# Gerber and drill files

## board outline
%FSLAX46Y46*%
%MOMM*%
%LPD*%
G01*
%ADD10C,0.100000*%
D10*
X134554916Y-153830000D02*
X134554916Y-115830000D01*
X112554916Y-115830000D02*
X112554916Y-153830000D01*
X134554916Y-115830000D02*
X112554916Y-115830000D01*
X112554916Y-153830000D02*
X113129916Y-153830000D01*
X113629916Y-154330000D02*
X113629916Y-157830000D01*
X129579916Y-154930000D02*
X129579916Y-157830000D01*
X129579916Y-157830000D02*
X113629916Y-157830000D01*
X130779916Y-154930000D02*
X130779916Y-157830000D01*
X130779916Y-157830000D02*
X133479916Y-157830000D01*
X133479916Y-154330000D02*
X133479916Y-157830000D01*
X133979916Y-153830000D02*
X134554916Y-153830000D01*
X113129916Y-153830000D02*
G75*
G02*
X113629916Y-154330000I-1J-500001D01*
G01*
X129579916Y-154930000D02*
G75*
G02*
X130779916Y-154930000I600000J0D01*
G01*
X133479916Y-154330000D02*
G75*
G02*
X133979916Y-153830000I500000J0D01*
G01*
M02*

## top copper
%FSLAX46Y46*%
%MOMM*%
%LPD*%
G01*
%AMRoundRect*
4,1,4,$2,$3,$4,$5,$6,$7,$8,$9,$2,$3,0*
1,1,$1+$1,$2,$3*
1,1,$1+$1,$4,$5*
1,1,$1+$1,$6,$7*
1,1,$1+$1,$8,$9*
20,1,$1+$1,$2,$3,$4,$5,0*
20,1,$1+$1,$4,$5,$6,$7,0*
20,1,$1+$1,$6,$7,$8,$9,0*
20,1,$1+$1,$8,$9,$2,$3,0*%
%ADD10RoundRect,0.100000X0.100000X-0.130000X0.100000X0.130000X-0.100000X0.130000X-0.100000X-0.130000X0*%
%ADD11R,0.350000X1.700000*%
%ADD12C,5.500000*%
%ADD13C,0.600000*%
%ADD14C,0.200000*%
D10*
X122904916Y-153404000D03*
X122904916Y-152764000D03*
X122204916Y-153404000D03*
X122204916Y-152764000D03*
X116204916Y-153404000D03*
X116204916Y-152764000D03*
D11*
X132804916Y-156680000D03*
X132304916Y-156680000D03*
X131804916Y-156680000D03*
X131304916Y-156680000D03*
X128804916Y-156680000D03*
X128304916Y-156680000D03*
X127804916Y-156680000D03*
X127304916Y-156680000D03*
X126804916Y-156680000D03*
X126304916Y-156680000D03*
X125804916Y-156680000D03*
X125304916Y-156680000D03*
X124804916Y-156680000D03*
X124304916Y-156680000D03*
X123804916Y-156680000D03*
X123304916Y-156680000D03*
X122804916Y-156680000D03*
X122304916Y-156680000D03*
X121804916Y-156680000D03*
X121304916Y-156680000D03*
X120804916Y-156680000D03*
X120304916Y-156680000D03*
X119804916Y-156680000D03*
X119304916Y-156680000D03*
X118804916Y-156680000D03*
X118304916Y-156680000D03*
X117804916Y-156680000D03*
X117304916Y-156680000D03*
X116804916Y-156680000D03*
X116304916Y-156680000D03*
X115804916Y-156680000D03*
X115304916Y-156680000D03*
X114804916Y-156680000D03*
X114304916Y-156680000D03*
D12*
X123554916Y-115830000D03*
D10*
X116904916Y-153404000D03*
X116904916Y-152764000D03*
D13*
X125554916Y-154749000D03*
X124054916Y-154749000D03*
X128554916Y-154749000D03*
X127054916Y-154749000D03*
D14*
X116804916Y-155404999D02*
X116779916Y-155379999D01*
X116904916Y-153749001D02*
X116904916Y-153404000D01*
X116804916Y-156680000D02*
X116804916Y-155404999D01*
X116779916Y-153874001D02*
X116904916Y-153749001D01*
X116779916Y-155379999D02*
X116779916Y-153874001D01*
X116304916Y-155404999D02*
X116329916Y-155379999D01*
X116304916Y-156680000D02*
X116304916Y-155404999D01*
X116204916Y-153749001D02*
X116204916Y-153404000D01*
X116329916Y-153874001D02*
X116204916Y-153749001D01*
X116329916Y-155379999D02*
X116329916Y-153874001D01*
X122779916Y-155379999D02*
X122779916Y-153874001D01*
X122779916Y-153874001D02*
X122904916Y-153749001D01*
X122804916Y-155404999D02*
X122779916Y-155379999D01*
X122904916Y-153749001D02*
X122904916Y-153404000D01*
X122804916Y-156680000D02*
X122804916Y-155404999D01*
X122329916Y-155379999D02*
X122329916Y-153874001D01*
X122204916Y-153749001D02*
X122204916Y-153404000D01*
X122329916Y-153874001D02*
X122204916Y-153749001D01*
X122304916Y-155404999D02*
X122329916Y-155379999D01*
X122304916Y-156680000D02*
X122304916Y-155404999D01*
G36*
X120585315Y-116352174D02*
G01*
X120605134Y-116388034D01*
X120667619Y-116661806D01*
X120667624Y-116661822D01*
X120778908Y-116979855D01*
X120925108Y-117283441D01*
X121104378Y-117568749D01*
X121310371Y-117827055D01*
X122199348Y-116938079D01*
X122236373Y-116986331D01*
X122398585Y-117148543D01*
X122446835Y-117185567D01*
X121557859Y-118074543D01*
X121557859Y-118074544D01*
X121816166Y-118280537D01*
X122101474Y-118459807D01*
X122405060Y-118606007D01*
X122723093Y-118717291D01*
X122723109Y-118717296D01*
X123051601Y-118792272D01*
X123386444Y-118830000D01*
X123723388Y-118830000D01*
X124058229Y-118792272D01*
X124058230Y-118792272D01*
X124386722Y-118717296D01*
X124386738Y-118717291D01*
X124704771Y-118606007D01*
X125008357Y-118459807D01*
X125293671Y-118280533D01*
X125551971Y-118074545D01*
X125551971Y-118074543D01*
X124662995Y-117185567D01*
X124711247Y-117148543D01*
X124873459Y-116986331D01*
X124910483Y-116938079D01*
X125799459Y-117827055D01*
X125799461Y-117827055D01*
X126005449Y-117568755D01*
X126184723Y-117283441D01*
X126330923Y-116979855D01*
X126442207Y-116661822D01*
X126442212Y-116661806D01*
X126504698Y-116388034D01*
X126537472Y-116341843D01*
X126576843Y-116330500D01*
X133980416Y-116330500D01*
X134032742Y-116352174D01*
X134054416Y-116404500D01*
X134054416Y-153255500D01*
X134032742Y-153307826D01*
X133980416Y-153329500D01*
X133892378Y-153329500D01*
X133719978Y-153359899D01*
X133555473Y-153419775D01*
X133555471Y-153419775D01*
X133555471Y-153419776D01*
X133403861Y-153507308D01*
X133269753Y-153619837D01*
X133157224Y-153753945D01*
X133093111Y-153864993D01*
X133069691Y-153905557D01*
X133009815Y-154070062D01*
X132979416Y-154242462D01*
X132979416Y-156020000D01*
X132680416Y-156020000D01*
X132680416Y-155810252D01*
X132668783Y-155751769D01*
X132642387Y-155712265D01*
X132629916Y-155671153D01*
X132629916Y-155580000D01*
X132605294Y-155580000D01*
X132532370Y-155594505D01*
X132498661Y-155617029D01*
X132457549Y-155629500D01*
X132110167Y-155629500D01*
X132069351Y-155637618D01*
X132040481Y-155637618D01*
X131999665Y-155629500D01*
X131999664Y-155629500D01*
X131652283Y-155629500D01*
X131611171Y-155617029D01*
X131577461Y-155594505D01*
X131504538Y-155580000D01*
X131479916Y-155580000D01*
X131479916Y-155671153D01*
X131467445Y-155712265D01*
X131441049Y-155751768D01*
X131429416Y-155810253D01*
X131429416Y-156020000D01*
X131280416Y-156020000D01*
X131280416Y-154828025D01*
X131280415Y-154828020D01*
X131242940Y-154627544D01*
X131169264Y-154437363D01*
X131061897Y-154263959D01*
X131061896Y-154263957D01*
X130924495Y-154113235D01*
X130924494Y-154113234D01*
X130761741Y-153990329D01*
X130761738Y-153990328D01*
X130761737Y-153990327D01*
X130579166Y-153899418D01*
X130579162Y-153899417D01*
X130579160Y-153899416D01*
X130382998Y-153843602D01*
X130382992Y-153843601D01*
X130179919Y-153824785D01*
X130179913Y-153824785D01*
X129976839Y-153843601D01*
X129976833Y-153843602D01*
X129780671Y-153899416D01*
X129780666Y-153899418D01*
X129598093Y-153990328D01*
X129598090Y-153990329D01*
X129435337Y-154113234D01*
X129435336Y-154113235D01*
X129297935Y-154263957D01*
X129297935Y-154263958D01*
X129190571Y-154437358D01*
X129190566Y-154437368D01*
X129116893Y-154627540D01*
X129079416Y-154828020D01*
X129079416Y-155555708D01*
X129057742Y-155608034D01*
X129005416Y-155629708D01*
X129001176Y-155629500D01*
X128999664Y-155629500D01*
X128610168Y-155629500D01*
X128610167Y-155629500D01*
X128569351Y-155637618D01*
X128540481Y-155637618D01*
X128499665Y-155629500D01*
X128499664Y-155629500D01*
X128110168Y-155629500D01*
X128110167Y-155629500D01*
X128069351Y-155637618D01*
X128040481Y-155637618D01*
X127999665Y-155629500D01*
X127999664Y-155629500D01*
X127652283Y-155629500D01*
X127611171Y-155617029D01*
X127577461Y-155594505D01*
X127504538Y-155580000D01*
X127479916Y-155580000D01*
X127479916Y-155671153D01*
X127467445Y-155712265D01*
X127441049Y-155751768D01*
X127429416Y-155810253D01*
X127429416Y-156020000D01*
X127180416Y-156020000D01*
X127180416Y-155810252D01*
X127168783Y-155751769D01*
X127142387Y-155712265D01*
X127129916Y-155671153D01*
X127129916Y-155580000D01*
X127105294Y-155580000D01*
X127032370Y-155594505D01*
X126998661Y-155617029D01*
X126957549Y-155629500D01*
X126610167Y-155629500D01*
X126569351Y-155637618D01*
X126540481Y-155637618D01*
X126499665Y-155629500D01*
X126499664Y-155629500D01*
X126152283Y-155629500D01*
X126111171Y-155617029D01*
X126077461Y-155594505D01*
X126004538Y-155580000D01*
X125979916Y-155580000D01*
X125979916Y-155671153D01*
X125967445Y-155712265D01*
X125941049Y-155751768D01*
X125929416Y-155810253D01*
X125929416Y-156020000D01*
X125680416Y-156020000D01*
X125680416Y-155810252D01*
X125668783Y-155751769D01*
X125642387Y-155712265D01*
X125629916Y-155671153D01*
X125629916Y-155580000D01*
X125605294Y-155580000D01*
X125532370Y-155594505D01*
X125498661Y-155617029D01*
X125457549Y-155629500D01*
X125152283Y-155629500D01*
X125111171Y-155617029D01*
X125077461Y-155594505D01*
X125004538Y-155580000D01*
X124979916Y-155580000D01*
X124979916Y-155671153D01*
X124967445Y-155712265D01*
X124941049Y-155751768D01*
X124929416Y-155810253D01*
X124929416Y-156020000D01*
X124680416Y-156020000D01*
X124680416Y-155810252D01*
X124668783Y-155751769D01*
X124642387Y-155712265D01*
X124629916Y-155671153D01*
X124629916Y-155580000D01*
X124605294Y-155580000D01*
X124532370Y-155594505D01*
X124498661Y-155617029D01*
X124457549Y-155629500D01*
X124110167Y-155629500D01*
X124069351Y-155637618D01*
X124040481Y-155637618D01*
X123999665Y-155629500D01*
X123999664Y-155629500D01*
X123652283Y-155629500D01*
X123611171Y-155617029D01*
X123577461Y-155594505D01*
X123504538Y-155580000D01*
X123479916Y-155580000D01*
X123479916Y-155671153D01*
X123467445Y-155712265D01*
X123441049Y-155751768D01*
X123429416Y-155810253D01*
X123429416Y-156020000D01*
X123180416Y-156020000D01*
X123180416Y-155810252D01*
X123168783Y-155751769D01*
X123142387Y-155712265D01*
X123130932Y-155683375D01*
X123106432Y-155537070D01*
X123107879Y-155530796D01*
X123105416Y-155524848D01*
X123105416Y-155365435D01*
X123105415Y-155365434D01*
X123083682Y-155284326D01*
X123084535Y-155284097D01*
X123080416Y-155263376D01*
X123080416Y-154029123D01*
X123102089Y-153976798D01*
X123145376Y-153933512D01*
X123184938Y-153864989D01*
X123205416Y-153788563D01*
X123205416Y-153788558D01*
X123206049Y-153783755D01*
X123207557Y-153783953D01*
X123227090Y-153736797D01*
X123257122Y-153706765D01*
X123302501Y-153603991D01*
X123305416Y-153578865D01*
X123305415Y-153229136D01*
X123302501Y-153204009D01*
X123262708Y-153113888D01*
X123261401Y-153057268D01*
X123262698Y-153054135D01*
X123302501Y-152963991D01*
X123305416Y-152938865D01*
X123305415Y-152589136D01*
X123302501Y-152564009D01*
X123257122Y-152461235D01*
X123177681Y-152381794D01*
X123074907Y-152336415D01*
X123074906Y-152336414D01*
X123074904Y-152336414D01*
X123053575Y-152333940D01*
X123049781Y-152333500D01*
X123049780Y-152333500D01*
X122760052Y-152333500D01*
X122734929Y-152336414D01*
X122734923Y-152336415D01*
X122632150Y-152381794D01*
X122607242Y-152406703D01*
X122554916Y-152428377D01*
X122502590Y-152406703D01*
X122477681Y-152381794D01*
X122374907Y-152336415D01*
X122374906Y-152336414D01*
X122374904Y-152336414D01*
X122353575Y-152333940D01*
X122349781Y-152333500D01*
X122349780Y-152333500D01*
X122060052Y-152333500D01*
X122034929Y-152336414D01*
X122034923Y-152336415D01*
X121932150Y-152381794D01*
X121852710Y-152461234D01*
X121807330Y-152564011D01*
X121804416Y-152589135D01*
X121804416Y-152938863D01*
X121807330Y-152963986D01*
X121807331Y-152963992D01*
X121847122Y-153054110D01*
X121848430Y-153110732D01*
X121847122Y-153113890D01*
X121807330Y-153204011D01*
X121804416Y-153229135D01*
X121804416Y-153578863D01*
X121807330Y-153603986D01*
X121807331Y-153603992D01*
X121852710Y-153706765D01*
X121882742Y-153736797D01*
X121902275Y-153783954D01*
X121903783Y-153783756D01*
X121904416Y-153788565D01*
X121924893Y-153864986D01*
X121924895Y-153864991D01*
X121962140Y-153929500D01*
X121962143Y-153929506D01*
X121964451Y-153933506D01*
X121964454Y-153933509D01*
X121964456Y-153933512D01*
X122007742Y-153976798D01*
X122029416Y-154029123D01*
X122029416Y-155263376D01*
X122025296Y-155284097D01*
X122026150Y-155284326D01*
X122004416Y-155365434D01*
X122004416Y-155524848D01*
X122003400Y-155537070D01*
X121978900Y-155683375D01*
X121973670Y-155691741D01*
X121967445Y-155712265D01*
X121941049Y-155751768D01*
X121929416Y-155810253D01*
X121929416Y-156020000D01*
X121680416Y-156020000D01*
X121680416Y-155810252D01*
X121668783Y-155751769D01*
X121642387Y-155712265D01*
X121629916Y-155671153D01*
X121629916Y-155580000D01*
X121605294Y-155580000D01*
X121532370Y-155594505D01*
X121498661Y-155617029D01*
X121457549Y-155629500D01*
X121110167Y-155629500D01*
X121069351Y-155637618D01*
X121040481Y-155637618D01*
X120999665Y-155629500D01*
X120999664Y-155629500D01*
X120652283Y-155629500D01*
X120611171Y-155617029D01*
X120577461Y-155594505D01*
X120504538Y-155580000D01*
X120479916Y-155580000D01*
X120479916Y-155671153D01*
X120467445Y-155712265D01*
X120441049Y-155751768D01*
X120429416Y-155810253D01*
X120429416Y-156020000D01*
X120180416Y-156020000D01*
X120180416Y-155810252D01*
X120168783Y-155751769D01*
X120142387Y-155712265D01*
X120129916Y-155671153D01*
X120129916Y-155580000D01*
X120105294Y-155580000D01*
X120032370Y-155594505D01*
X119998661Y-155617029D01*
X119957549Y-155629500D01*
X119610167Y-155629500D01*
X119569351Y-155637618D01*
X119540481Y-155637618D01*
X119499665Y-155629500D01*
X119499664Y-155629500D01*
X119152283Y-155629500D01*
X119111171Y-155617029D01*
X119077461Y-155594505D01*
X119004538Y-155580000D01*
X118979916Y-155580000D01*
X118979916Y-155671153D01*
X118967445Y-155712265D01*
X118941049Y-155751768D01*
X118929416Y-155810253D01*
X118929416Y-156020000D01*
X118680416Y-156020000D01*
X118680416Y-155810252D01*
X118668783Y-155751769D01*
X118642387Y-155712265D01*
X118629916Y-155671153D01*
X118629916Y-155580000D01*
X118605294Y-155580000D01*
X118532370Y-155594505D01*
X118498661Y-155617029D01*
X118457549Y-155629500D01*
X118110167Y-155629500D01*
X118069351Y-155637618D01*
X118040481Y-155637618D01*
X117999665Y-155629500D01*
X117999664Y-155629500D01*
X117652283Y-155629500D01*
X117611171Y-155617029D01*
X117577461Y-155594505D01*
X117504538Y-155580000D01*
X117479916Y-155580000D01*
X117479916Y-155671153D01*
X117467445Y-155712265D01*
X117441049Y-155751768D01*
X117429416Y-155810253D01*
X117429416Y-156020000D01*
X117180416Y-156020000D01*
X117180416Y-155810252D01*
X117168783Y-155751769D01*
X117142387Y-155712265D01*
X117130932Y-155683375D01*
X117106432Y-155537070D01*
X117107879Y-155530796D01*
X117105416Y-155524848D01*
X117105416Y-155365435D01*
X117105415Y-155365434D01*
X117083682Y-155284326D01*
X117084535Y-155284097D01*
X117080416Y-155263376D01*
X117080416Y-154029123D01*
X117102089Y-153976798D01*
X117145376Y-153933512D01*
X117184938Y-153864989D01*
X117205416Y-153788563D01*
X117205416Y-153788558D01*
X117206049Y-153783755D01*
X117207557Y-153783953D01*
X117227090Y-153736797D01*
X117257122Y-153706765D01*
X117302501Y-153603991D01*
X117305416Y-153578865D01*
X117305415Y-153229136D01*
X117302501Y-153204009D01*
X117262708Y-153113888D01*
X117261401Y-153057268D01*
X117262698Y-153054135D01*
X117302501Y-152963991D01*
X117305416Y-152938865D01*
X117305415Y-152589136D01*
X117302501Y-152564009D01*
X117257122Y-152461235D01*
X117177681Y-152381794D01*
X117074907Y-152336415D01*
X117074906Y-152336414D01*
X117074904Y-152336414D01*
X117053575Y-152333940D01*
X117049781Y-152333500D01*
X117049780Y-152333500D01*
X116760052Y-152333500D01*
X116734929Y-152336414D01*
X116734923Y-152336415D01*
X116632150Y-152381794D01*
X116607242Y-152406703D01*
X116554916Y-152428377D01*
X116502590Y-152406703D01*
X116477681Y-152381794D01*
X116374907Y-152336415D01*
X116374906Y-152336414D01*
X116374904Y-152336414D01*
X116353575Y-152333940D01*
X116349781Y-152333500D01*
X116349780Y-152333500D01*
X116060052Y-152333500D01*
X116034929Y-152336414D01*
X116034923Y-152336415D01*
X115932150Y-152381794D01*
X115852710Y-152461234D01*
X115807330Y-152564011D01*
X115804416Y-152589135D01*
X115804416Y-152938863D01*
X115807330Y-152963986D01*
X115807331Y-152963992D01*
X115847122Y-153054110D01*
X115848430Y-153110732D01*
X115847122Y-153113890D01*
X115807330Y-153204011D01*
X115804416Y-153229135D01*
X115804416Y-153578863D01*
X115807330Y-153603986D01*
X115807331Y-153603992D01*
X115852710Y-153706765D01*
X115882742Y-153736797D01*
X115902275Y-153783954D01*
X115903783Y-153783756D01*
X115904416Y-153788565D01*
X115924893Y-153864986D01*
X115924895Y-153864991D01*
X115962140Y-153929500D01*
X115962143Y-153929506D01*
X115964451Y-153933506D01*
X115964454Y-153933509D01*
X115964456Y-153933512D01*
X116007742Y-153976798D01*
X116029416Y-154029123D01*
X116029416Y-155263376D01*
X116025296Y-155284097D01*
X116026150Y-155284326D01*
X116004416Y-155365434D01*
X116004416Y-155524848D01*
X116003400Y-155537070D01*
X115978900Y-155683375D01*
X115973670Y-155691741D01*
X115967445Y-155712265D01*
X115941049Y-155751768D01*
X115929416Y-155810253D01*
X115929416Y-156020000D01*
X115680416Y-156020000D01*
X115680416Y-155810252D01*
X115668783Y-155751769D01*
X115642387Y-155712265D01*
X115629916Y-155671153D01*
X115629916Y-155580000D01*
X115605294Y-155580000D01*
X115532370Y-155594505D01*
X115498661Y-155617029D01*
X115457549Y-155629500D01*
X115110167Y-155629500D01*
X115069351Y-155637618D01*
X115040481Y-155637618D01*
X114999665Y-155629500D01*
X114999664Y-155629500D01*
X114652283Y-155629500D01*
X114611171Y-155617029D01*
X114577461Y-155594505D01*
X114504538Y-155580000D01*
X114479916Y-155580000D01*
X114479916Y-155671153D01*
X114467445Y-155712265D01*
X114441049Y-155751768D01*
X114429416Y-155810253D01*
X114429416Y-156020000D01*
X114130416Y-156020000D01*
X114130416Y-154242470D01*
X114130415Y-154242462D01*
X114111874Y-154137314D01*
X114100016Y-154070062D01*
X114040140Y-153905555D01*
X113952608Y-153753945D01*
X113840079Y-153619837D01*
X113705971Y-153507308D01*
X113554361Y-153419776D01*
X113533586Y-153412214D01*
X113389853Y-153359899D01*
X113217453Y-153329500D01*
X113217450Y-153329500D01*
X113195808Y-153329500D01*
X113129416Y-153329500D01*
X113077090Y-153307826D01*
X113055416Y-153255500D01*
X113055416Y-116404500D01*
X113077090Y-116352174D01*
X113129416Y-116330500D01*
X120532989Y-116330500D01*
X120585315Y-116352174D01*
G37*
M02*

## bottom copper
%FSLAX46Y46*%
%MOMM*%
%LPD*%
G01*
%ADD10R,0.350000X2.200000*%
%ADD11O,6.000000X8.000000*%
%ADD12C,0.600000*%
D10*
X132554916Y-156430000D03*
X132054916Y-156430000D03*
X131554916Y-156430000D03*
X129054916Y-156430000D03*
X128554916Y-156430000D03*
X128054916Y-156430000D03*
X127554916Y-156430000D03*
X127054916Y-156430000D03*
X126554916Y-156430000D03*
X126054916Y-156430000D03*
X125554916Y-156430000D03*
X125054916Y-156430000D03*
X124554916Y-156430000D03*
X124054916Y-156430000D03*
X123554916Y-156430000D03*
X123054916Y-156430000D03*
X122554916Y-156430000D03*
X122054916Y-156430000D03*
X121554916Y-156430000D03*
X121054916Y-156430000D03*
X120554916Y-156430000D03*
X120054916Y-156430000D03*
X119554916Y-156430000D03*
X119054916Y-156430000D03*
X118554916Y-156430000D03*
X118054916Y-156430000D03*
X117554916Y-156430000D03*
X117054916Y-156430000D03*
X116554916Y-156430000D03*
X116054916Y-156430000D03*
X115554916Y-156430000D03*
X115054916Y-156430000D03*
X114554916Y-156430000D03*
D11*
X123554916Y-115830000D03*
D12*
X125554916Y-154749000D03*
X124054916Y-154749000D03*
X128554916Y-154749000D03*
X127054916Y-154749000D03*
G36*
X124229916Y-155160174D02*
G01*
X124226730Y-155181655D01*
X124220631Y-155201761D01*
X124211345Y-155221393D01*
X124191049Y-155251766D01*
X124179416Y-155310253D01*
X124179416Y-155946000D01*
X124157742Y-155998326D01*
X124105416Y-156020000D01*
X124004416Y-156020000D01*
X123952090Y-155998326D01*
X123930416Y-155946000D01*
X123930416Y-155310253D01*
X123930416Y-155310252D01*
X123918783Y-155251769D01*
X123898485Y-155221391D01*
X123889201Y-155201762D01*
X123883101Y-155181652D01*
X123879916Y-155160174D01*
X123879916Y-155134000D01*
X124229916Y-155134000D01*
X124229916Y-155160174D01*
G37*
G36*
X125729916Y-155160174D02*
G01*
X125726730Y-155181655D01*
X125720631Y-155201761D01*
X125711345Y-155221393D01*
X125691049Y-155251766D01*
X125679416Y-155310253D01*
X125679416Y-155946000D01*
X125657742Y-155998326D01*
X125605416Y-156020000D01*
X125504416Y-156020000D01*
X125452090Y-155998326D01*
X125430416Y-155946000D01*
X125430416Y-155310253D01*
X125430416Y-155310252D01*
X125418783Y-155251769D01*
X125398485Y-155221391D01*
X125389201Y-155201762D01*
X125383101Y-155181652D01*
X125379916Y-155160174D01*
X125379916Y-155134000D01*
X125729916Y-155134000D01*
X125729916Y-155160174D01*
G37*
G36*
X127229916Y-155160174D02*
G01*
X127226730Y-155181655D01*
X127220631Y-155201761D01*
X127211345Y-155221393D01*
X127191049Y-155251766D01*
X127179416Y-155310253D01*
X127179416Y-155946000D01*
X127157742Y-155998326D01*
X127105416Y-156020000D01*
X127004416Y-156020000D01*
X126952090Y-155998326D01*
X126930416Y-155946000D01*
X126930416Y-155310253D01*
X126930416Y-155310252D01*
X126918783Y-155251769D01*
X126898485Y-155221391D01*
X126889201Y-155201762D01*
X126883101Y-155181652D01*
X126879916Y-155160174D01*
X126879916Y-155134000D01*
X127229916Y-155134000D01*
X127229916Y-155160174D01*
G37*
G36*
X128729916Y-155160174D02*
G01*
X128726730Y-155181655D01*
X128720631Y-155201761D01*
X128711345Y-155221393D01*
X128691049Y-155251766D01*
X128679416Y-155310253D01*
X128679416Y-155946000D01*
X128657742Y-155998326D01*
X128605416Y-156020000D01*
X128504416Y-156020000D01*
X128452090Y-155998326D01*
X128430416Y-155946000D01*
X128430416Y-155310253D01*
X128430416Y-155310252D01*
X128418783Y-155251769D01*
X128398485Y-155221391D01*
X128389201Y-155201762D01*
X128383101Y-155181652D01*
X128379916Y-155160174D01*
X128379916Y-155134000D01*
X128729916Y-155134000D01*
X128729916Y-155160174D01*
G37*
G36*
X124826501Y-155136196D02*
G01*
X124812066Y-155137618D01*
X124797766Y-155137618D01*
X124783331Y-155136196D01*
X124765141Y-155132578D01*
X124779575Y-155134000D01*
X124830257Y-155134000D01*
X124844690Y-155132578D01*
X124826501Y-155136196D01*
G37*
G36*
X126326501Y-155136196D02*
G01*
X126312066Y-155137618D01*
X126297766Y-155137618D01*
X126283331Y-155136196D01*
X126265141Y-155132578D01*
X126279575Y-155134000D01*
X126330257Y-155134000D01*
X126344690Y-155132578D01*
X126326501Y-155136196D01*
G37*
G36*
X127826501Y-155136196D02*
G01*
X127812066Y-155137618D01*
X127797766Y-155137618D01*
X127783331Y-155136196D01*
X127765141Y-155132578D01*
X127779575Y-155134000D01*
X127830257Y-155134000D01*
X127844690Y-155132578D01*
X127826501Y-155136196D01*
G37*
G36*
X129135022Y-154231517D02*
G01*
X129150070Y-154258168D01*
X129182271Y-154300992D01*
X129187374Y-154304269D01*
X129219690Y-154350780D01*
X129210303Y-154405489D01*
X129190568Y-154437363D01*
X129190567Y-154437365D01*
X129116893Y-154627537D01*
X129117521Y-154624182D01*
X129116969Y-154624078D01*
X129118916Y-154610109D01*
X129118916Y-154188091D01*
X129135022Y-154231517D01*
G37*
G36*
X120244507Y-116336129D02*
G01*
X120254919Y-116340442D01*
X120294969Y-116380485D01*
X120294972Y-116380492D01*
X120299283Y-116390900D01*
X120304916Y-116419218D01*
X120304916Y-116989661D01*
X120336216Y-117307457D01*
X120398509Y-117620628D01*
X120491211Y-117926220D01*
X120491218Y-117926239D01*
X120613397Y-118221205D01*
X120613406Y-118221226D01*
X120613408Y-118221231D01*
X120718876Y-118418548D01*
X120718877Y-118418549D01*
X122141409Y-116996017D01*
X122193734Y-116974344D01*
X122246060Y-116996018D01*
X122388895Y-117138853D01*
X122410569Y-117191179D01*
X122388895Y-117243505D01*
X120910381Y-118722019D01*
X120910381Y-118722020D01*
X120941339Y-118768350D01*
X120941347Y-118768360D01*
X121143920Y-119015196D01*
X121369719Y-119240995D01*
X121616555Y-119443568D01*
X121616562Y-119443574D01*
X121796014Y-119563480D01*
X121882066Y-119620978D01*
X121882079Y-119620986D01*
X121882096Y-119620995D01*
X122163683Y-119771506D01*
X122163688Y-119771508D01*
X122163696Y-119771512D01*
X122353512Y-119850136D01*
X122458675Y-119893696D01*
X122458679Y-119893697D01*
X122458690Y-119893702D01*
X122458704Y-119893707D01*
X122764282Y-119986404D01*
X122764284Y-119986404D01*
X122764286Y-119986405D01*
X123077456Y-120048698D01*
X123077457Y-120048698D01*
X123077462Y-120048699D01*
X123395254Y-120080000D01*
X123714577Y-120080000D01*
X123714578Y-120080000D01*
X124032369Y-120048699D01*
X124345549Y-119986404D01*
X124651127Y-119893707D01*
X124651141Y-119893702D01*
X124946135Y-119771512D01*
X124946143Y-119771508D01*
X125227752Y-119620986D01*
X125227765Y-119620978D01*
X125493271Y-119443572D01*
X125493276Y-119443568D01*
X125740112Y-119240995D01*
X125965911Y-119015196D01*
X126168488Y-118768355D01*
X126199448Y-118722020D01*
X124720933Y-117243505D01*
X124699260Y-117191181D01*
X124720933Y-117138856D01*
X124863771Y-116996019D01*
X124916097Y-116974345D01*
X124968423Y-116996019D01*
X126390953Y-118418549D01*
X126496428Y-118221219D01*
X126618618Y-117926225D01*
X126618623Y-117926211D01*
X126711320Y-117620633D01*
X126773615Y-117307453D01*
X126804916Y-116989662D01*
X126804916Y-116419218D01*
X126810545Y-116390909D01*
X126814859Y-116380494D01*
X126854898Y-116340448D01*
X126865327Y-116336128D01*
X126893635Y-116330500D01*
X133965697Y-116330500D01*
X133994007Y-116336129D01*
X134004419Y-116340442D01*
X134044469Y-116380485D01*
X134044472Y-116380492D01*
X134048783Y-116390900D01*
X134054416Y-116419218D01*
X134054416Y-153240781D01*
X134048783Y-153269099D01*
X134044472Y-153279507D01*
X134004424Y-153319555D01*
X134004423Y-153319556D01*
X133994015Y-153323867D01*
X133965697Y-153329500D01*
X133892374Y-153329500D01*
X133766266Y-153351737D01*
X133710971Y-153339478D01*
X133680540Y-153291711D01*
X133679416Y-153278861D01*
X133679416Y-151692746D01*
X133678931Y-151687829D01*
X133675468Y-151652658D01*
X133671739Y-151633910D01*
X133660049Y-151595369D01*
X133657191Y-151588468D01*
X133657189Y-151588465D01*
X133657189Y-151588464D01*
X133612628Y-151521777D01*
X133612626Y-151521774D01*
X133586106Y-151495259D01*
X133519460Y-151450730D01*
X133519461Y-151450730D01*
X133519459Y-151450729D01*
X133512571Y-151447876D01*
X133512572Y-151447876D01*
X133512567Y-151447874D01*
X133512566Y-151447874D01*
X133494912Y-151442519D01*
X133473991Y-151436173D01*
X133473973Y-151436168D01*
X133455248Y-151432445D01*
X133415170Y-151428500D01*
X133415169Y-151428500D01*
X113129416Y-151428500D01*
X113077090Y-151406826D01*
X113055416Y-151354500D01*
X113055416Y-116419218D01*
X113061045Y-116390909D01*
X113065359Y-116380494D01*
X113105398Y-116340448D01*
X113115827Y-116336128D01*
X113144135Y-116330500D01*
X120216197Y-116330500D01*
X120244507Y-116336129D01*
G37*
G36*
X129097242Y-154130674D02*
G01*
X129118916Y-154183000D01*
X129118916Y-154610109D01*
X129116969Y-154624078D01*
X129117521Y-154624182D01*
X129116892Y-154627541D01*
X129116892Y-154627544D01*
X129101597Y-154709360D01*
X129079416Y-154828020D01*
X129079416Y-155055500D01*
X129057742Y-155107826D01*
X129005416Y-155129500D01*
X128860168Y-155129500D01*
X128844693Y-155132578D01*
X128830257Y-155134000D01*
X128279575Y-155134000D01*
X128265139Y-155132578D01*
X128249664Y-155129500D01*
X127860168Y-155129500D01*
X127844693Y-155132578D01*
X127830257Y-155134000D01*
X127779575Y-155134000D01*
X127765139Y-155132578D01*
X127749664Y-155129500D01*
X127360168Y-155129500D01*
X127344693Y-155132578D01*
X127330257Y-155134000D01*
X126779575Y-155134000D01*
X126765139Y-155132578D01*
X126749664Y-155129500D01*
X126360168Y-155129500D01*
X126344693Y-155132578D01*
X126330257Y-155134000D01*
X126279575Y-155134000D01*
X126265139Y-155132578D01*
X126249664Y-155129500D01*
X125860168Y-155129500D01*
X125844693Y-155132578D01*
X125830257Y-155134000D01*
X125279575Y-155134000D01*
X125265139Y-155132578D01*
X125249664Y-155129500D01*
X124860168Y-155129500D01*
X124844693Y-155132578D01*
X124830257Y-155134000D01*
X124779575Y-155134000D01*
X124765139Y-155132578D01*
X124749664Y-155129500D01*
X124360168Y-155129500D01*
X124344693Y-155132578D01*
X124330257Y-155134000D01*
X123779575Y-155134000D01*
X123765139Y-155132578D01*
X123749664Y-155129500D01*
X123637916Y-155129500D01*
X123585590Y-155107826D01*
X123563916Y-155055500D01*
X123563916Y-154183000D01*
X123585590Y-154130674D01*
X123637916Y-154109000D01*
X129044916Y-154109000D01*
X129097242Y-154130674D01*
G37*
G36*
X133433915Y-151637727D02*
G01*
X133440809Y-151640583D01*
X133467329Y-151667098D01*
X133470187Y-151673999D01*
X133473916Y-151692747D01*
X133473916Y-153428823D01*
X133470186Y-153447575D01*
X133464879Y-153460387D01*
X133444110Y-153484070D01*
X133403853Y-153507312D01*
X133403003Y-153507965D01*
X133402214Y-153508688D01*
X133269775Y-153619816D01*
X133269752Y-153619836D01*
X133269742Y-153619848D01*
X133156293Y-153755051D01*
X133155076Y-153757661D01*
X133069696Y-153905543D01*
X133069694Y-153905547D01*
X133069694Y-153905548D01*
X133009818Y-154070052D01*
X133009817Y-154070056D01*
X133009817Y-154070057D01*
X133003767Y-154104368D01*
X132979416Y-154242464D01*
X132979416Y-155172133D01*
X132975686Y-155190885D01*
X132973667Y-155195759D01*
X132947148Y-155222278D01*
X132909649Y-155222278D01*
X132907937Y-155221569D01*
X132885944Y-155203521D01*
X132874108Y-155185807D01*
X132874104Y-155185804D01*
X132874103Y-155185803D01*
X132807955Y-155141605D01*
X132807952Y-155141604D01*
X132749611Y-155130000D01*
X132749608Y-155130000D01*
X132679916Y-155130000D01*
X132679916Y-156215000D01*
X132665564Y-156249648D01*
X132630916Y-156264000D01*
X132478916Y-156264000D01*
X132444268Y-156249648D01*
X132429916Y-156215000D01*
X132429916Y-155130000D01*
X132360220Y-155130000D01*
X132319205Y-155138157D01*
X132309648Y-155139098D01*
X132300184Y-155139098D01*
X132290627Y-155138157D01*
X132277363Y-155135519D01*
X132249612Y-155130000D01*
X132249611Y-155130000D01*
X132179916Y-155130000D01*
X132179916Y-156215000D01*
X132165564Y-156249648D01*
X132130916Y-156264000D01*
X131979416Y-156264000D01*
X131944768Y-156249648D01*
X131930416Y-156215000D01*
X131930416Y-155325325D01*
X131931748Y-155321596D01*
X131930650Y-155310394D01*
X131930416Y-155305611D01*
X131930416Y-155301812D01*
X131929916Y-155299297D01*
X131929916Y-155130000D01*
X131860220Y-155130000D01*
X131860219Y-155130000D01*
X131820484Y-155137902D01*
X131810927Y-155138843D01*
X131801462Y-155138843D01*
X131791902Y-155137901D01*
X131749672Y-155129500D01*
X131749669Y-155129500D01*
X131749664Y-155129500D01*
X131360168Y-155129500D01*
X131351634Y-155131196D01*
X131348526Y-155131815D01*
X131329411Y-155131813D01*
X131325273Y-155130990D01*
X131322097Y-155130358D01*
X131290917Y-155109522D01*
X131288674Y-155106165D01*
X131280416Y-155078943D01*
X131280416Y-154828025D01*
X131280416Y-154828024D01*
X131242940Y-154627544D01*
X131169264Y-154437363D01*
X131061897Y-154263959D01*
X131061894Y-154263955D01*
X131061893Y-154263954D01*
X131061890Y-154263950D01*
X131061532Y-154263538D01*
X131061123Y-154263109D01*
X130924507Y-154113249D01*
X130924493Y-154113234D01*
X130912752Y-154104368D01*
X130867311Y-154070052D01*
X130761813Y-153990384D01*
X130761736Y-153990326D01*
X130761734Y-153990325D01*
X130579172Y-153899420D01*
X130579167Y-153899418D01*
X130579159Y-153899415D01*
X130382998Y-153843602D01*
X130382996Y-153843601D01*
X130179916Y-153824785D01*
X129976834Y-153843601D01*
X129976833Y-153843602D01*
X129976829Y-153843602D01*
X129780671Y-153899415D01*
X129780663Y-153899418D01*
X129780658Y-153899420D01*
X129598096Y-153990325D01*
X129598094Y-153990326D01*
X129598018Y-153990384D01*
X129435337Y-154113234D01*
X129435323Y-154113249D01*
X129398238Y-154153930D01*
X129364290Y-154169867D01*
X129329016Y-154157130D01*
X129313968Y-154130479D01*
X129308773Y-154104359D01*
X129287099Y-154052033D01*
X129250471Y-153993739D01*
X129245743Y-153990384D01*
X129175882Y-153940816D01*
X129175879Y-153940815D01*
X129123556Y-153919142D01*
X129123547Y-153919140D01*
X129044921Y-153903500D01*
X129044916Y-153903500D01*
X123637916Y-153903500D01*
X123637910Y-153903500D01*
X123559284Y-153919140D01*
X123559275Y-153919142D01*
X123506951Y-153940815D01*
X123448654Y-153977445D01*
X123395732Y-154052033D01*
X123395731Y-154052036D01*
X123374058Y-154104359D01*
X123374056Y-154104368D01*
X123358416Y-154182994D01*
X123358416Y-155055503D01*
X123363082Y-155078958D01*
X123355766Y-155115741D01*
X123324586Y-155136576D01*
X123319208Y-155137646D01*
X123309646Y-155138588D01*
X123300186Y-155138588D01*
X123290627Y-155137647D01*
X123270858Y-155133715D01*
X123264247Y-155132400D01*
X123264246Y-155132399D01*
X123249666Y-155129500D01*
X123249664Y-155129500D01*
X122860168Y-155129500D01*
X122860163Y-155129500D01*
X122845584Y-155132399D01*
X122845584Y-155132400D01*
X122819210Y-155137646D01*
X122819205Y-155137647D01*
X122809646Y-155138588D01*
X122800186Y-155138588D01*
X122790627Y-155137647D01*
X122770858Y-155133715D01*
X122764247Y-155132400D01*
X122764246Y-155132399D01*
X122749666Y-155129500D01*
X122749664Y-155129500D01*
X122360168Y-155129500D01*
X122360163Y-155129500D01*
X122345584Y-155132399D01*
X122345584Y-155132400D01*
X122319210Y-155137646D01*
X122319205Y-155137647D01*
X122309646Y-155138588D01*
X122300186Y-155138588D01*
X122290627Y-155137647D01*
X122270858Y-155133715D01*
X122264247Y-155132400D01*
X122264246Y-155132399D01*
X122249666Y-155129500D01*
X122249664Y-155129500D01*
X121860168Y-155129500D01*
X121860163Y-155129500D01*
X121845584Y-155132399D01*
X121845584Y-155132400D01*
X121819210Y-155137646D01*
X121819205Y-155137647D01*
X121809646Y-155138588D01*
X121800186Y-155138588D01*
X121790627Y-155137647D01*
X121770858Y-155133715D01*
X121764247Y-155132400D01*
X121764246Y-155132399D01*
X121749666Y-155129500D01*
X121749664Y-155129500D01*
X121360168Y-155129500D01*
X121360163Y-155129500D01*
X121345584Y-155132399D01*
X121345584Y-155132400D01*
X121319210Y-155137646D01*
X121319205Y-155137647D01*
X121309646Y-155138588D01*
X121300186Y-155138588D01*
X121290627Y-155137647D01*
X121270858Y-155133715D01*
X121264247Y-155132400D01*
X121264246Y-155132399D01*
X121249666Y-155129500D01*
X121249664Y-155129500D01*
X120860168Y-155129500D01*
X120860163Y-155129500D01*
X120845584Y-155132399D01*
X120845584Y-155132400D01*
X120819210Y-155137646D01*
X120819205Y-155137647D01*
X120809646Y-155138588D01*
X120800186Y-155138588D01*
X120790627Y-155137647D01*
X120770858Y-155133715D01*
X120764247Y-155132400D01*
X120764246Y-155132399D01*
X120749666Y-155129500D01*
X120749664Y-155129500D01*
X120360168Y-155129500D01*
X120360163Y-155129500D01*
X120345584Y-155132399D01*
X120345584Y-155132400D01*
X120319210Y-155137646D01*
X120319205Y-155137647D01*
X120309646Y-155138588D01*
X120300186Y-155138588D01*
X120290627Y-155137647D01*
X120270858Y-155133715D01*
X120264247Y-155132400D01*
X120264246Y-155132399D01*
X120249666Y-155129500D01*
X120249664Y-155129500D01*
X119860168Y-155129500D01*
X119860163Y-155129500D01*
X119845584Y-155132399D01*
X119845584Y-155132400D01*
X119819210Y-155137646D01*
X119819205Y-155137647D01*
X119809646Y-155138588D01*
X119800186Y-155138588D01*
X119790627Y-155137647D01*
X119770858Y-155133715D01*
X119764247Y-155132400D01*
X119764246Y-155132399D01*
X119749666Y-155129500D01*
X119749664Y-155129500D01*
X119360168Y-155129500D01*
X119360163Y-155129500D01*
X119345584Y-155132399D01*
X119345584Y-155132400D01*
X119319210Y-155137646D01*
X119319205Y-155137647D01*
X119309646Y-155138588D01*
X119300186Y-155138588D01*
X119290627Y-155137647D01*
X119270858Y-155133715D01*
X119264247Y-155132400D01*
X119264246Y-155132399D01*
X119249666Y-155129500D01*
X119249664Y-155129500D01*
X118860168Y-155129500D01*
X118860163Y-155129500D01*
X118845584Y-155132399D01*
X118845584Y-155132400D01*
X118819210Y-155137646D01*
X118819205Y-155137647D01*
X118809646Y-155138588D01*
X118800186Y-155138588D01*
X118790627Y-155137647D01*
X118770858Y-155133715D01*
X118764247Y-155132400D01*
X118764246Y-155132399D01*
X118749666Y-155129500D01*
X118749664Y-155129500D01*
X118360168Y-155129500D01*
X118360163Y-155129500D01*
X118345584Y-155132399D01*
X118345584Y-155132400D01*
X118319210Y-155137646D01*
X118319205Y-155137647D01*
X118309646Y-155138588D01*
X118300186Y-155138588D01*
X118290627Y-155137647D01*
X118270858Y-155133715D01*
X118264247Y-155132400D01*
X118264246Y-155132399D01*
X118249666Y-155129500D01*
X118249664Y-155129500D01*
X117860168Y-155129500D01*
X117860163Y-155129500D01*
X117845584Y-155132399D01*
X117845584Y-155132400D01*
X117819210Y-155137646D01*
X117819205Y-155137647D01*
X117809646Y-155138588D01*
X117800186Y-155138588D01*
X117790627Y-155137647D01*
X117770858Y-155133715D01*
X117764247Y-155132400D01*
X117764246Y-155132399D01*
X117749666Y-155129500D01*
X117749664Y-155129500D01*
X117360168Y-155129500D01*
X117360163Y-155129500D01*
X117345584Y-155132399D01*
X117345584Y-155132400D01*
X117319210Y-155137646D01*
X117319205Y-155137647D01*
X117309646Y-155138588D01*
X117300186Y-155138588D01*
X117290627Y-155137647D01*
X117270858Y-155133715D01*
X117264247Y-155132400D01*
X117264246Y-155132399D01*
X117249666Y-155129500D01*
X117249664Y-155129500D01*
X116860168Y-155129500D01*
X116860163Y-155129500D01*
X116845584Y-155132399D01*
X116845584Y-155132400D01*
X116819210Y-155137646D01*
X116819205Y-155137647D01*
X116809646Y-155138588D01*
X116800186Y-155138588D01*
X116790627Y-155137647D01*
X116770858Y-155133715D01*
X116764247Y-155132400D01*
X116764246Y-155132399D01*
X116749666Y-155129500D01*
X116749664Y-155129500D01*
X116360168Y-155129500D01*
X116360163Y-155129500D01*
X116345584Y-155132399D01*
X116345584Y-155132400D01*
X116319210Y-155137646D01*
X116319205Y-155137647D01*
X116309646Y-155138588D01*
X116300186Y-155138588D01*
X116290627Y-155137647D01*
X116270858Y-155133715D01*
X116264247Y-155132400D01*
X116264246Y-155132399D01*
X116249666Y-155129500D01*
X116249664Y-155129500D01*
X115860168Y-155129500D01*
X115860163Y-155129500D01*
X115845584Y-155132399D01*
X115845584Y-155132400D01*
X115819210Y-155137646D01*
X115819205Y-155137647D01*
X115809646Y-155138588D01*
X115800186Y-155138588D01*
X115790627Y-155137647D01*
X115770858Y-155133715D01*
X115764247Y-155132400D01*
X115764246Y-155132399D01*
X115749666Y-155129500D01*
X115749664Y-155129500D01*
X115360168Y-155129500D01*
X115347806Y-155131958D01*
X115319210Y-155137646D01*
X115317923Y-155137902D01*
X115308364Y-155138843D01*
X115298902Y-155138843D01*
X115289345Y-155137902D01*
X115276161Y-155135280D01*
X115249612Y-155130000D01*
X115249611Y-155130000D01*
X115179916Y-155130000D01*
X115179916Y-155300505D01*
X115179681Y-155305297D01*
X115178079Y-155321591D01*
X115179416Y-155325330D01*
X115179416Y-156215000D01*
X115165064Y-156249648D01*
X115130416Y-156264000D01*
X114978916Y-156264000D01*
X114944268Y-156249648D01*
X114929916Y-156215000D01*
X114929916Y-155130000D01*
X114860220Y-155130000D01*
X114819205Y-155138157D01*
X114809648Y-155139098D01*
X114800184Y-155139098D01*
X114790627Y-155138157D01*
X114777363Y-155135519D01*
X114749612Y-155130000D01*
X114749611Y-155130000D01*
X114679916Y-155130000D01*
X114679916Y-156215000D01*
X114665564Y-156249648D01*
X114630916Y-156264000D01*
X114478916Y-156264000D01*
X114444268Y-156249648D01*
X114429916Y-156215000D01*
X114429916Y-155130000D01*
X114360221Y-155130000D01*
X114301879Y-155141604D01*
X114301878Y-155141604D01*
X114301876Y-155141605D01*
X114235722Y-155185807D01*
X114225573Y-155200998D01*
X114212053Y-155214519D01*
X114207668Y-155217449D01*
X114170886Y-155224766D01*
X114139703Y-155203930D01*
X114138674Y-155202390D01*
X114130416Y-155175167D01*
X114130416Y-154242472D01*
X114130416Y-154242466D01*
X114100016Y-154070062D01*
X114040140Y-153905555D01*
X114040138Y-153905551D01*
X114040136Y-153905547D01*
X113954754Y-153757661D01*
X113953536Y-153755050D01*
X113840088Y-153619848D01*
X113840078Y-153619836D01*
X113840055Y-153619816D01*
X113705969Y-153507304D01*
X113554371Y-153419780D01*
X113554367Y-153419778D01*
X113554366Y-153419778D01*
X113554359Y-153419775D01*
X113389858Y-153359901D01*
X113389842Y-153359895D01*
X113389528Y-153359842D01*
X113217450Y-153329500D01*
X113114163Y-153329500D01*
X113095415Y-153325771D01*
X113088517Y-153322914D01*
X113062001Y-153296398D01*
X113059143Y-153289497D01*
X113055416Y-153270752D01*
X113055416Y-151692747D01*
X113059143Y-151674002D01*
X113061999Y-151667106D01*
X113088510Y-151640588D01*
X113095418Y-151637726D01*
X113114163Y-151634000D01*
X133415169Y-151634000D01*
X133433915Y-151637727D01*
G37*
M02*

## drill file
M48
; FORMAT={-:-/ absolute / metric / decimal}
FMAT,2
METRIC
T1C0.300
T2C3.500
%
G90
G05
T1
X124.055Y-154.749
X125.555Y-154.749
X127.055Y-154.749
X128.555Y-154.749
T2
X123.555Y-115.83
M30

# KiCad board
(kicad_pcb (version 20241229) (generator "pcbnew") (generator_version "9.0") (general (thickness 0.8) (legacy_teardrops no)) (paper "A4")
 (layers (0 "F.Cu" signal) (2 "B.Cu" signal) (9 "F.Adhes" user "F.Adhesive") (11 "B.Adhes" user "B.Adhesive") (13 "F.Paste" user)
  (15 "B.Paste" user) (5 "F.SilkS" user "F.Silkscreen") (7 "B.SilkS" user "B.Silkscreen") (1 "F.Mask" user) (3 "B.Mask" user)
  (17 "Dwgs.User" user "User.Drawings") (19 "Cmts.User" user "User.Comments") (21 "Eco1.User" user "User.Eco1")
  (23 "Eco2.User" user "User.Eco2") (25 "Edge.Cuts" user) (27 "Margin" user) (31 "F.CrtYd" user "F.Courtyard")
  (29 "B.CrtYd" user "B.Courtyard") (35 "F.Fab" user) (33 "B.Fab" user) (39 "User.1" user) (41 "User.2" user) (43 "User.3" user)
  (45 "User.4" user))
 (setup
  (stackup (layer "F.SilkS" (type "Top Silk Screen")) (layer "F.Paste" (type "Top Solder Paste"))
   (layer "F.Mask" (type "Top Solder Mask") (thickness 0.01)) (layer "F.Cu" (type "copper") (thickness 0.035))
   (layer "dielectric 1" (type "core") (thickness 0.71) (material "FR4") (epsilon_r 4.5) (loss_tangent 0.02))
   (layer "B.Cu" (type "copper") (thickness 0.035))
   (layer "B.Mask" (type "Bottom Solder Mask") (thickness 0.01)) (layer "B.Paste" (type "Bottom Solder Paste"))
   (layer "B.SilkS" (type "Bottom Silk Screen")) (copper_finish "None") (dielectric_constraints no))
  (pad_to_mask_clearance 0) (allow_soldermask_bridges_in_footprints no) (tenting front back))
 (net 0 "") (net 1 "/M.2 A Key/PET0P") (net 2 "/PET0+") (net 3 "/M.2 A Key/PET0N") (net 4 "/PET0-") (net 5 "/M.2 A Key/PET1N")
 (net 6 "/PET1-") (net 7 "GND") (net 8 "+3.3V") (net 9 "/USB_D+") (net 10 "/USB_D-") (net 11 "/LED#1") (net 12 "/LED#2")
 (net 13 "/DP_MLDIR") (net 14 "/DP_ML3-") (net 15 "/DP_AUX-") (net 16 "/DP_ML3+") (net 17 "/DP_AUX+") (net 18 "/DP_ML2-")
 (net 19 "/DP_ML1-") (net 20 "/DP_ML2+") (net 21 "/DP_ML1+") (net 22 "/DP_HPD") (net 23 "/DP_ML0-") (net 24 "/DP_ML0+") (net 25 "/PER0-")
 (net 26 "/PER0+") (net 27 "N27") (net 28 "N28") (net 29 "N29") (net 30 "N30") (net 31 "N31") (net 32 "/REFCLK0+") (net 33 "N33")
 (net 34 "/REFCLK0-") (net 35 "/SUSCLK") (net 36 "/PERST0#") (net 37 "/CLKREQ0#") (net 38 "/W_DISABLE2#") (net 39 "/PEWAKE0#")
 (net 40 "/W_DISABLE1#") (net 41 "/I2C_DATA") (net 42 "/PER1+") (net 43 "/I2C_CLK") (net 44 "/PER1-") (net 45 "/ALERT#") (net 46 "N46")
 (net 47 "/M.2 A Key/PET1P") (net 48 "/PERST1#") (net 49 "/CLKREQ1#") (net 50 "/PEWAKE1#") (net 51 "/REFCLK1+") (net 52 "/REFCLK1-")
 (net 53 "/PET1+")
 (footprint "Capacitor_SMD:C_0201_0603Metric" (layer "F.Cu") (at 122.904916 153.084 90)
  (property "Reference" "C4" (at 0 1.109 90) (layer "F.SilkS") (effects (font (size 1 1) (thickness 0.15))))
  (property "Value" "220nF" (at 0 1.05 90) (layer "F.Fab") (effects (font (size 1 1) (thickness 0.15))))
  (pad "" smd roundrect (at -0.345 0 90) (size 0.318 0.36) (layers "F.Paste") (roundrect_rratio 0.25))
  (pad "" smd roundrect (at 0.345 0 90) (size 0.318 0.36) (layers "F.Paste") (roundrect_rratio 0.25))
  (pad "1" smd roundrect (at -0.32 0 90) (size 0.46 0.4) (layers "F.Cu" "F.Mask") (roundrect_rratio 0.25) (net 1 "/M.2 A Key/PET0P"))
  (pad "2" smd roundrect (at 0.32 0 90) (size 0.46 0.4) (layers "F.Cu" "F.Mask") (roundrect_rratio 0.25) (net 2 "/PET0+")))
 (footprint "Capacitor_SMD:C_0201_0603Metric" (layer "F.Cu") (at 122.204916 153.084 90)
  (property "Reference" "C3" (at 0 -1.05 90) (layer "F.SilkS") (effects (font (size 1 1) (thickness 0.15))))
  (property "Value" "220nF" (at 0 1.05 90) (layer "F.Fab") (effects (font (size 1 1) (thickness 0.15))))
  (pad "" smd roundrect (at -0.345 0 90) (size 0.318 0.36) (layers "F.Paste") (roundrect_rratio 0.25))
  (pad "" smd roundrect (at 0.345 0 90) (size 0.318 0.36) (layers "F.Paste") (roundrect_rratio 0.25))
  (pad "1" smd roundrect (at -0.32 0 90) (size 0.46 0.4) (layers "F.Cu" "F.Mask") (roundrect_rratio 0.25) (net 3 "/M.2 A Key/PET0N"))
  (pad "2" smd roundrect (at 0.32 0 90) (size 0.46 0.4) (layers "F.Cu" "F.Mask") (roundrect_rratio 0.25) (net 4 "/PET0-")))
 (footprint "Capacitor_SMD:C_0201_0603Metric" (layer "F.Cu") (at 116.204916 153.084 90)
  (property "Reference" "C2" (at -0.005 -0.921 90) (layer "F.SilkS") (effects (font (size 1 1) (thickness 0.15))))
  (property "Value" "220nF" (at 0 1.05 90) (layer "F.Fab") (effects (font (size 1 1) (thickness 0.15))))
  (pad "" smd roundrect (at -0.345 0 90) (size 0.318 0.36) (layers "F.Paste") (roundrect_rratio 0.25))
  (pad "" smd roundrect (at 0.345 0 90) (size 0.318 0.36) (layers "F.Paste") (roundrect_rratio 0.25))
  (pad "1" smd roundrect (at -0.32 0 90) (size 0.46 0.4) (layers "F.Cu" "F.Mask") (roundrect_rratio 0.25) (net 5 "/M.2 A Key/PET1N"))
  (pad "2" smd roundrect (at 0.32 0 90) (size 0.46 0.4) (layers "F.Cu" "F.Mask") (roundrect_rratio 0.25) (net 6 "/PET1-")))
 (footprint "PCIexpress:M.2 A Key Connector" (layer "F.Cu") (at 123.554916 156.72)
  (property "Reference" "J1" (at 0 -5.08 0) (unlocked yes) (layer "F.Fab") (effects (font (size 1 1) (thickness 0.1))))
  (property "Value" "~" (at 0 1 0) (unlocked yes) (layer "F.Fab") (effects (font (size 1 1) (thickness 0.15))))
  (fp_line (start -11 -2.89) (end -10.425 -2.89) (stroke (width 0.1) (type default)) (layer "Edge.Cuts"))
  (fp_line (start -9.925 -2.39) (end -9.925 1.11) (stroke (width 0.1) (type default)) (layer "Edge.Cuts"))
  (fp_line (start 6.025 -1.79) (end 6.025 1.11) (stroke (width 0.1) (type default)) (layer "Edge.Cuts"))
  (fp_line (start 6.025 1.11) (end -9.925 1.11) (stroke (width 0.1) (type default)) (layer "Edge.Cuts"))
  (fp_line (start 7.225 -1.79) (end 7.225 1.11) (stroke (width 0.1) (type default)) (layer "Edge.Cuts"))
  (fp_line (start 7.225 1.11) (end 9.925 1.11) (stroke (width 0.1) (type default)) (layer "Edge.Cuts"))
  (fp_line (start 9.925 -2.39) (end 9.925 1.11) (stroke (width 0.1) (type default)) (layer "Edge.Cuts"))
  (fp_line (start 10.425 -2.89) (end 11 -2.89) (stroke (width 0.1) (type default)) (layer "Edge.Cuts"))
  (fp_arc (start -10.425 -2.89) (mid -10.071447 -2.743553) (end -9.925 -2.39) (stroke (width 0.1) (type default)) (layer "Edge.Cuts"))
  (fp_arc (start 6.025 -1.79) (mid 6.625 -2.39) (end 7.225 -1.79) (stroke (width 0.1) (type default)) (layer "Edge.Cuts"))
  (fp_arc (start 9.925 -2.39) (mid 10.071447 -2.743553) (end 10.425 -2.89) (stroke (width 0.1) (type default)) (layer "Edge.Cuts"))
  (pad "1" smd rect (at 9.25 -0.04 180) (size 0.35 1.7) (layers "F.Cu") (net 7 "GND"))
  (pad "2" smd rect (at 9 -0.29 180) (size 0.35 2.2) (layers "B.Cu") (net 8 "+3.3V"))
  (pad "3" smd rect (at 8.75 -0.04 180) (size 0.35 1.7) (layers "F.Cu") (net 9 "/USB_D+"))
  (pad "4" smd rect (at 8.5 -0.29 180) (size 0.35 2.2) (layers "B.Cu") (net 8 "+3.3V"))
  (pad "5" smd rect (at 8.25 -0.04 180) (size 0.35 1.7) (layers "F.Cu") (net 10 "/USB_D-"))
  (pad "6" smd rect (at 8 -0.29 180) (size 0.35 2.2) (layers "B.Cu") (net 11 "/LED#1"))
  (pad "7" smd rect (at 7.75 -0.04 180) (size 0.35 1.7) (layers "F.Cu") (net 7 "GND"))
  (pad "16" smd rect (at 5.5 -0.29 180) (size 0.35 2.2) (layers "B.Cu") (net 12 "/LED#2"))
  (pad "17" smd rect (at 5.25 -0.04 180) (size 0.35 1.7) (layers "F.Cu") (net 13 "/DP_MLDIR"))
  (pad "18" smd rect (at 5 -0.29 180) (size 0.35 2.2) (layers "B.Cu") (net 7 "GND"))
  (pad "19" smd rect (at 4.75 -0.04 180) (size 0.35 1.7) (layers "F.Cu") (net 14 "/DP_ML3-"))
  (pad "20" smd rect (at 4.5 -0.29 180) (size 0.35 2.2) (layers "B.Cu") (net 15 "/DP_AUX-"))
  (pad "21" smd rect (at 4.25 -0.04 180) (size 0.35 1.7) (layers "F.Cu") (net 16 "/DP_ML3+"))
  (pad "22" smd rect (at 4 -0.29 180) (size 0.35 2.2) (layers "B.Cu") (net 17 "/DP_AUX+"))
  (pad "23" smd rect (at 3.75 -0.04 180) (size 0.35 1.7) (layers "F.Cu") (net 7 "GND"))
  (pad "24" smd rect (at 3.5 -0.29 180) (size 0.35 2.2) (layers "B.Cu") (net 7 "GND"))
  (pad "25" smd rect (at 3.25 -0.04 180) (size 0.35 1.7) (layers "F.Cu") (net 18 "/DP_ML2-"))
  (pad "26" smd rect (at 3 -0.29 180) (size 0.35 2.2) (layers "B.Cu") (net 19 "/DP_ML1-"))
  (pad "27" smd rect (at 2.75 -0.04 180) (size 0.35 1.7) (layers "F.Cu") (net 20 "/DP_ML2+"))
  (pad "28" smd rect (at 2.5 -0.29 180) (size 0.35 2.2) (layers "B.Cu") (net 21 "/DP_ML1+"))
  (pad "29" smd rect (at 2.25 -0.04 180) (size 0.35 1.7) (layers "F.Cu") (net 7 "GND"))
  (pad "30" smd rect (at 2 -0.29 180) (size 0.35 2.2) (layers "B.Cu") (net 7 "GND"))
  (pad "31" smd rect (at 1.75 -0.04 180) (size 0.35 1.7) (layers "F.Cu") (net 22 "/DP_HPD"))
  (pad "32" smd rect (at 1.5 -0.29 180) (size 0.35 2.2) (layers "B.Cu") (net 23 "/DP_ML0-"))
  (pad "33" smd rect (at 1.25 -0.04 180) (size 0.35 1.7) (layers "F.Cu") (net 7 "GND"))
  (pad "34" smd rect (at 1 -0.29 180) (size 0.35 2.2) (layers "B.Cu") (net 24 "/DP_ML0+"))
  (pad "35" smd rect (at 0.75 -0.04 180) (size 0.35 1.7) (layers "F.Cu") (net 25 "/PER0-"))
  (pad "36" smd rect (at 0.5 -0.29 180) (size 0.35 2.2) (layers "B.Cu") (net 7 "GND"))
  (pad "37" smd rect (at 0.25 -0.04 180) (size 0.35 1.7) (layers "F.Cu") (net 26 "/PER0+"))
  (pad "38" smd rect (at 0 -0.29 180) (size 0.35 2.2) (layers "B.Cu") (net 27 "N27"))
  (pad "39" smd rect (at -0.25 -0.04 180) (size 0.35 1.7) (layers "F.Cu") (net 7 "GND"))
  (pad "40" smd rect (at -0.5 -0.29 180) (size 0.35 2.2) (layers "B.Cu") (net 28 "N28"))
  (pad "41" smd rect (at -0.75 -0.04 180) (size 0.35 1.7) (layers "F.Cu") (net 1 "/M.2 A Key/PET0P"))
  (pad "42" smd rect (at -1 -0.29 180) (size 0.35 2.2) (layers "B.Cu") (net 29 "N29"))
  (pad "43" smd rect (at -1.25 -0.04 180) (size 0.35 1.7) (layers "F.Cu") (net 3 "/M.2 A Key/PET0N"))
  (pad "44" smd rect (at -1.5 -0.29 180) (size 0.35 2.2) (layers "B.Cu") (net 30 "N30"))
  (pad "45" smd rect (at -1.75 -0.04 180) (size 0.35 1.7) (layers "F.Cu") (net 7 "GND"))
  (pad "46" smd rect (at -2 -0.29 180) (size 0.35 2.2) (layers "B.Cu") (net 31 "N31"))
  (pad "47" smd rect (at -2.25 -0.04 180) (size 0.35 1.7) (layers "F.Cu") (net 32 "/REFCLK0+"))
  (pad "48" smd rect (at -2.5 -0.29 180) (size 0.35 2.2) (layers "B.Cu") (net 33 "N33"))
  (pad "49" smd rect (at -2.75 -0.04 180) (size 0.35 1.7) (layers "F.Cu") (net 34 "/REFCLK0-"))
  (pad "50" smd rect (at -3 -0.29 180) (size 0.35 2.2) (layers "B.Cu") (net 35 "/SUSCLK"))
  (pad "51" smd rect (at -3.25 -0.04 180) (size 0.35 1.7) (layers "F.Cu") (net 7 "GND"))
  (pad "52" smd rect (at -3.5 -0.29 180) (size 0.35 2.2) (layers "B.Cu") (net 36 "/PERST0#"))
  (pad "53" smd rect (at -3.75 -0.04 180) (size 0.35 1.7) (layers "F.Cu") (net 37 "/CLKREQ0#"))
  (pad "54" smd rect (at -4 -0.29 180) (size 0.35 2.2) (layers "B.Cu") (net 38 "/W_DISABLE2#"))
  (pad "55" smd rect (at -4.25 -0.04 180) (size 0.35 1.7) (layers "F.Cu") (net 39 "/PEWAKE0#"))
  (pad "56" smd rect (at -4.5 -0.29 180) (size 0.35 2.2) (layers "B.Cu") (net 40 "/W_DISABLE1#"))
  (pad "57" smd rect (at -4.75 -0.04 180) (size 0.35 1.7) (layers "F.Cu") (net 7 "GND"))
  (pad "58" smd rect (at -5 -0.29 180) (size 0.35 2.2) (layers "B.Cu") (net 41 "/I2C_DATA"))
  (pad "59" smd rect (at -5.25 -0.04 180) (size 0.35 1.7) (layers "F.Cu") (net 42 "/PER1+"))
  (pad "60" smd rect (at -5.5 -0.29 180) (size 0.35 2.2) (layers "B.Cu") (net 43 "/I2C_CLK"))
  (pad "61" smd rect (at -5.75 -0.04 180) (size 0.35 1.7) (layers "F.Cu") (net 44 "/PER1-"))
  (pad "62" smd rect (at -6 -0.29 180) (size 0.35 2.2) (layers "B.Cu") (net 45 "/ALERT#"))
  (pad "63" smd rect (at -6.25 -0.04 180) (size 0.35 1.7) (layers "F.Cu") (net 7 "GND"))
  (pad "64" smd rect (at -6.5 -0.29 180) (size 0.35 2.2) (layers "B.Cu") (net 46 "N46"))
  (pad "65" smd rect (at -6.75 -0.04 180) (size 0.35 1.7) (layers "F.Cu") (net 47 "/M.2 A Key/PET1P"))
  (pad "66" smd rect (at -7 -0.29 180) (size 0.35 2.2) (layers "B.Cu") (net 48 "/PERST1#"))
  (pad "67" smd rect (at -7.25 -0.04 180) (size 0.35 1.7) (layers "F.Cu") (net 5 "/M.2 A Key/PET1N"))
  (pad "68" smd rect (at -7.5 -0.29 180) (size 0.35 2.2) (layers "B.Cu") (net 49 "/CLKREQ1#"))
  (pad "69" smd rect (at -7.75 -0.04 180) (size 0.35 1.7) (layers "F.Cu") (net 7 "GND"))
  (pad "70" smd rect (at -8 -0.29 180) (size 0.35 2.2) (layers "B.Cu") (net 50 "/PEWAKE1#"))
  (pad "71" smd rect (at -8.25 -0.04 180) (size 0.35 1.7) (layers "F.Cu") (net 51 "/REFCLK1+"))
  (pad "72" smd rect (at -8.5 -0.29 180) (size 0.35 2.2) (layers "B.Cu") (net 8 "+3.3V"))
  (pad "73" smd rect (at -8.75 -0.04 180) (size 0.35 1.7) (layers "F.Cu") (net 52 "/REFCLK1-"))
  (pad "74" smd rect (at -9 -0.29 180) (size 0.35 2.2) (layers "B.Cu") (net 8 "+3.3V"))
  (pad "75" smd rect (at -9.25 -0.04 180) (size 0.35 1.7) (layers "F.Cu") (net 7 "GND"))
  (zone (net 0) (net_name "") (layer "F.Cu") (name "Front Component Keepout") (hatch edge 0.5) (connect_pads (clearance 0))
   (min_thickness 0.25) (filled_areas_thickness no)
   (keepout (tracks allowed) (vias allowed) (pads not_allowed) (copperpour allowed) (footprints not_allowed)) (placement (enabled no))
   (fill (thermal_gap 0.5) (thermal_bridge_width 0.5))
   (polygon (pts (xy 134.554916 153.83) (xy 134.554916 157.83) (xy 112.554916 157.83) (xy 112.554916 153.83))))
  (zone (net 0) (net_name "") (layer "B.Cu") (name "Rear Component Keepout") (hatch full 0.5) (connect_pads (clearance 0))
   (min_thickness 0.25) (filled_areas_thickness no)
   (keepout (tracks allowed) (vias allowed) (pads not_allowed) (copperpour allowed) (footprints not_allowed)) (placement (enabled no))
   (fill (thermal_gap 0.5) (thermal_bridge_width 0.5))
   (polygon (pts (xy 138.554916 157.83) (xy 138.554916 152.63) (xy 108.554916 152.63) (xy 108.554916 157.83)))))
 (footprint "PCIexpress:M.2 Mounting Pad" (layer "F.Cu") (at 123.554916 115.83)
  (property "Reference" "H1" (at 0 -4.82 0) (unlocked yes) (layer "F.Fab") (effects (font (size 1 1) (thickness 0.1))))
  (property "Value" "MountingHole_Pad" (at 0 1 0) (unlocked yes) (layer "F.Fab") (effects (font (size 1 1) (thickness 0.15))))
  (pad "1" thru_hole circle (at 0 0) (size 5.5 5.5) (drill 3.5) (layers "*.Cu" "*.Mask") (remove_unused_layers no) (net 7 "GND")
   (padstack (mode front_inner_back)
    (layer "Inner" (shape circle) (size 5.5 5.5) (zone_connect -1))
    (layer "B.Cu" (shape oval) (size 6 8) (thermal_bridge_angle 45) (zone_connect -1)))))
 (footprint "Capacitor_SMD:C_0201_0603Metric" (layer "F.Cu") (at 116.904916 153.084 90)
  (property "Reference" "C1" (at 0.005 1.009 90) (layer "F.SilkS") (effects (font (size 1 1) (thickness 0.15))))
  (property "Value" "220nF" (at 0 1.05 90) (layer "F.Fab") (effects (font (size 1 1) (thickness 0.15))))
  (pad "" smd roundrect (at -0.345 0 90) (size 0.318 0.36) (layers "F.Paste") (roundrect_rratio 0.25))
  (pad "" smd roundrect (at 0.345 0 90) (size 0.318 0.36) (layers "F.Paste") (roundrect_rratio 0.25))
  (pad "1" smd roundrect (at -0.32 0 90) (size 0.46 0.4) (layers "F.Cu" "F.Mask") (roundrect_rratio 0.25) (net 47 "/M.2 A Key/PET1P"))
  (pad "2" smd roundrect (at 0.32 0 90) (size 0.46 0.4) (layers "F.Cu" "F.Mask") (roundrect_rratio 0.25) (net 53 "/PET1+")))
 (gr_line (start 134.554916 153.83) (end 134.554916 115.83) (stroke (width 0.1) (type default)) (layer "Edge.Cuts"))
 (gr_line (start 112.554916 115.83) (end 112.554916 153.83) (stroke (width 0.1) (type default)) (layer "Edge.Cuts"))
 (gr_line (start 134.554916 115.83) (end 112.554916 115.83) (stroke (width 0.1) (type solid)) (layer "Edge.Cuts"))
 (via (at 125.554916 154.749) (size 0.6) (drill 0.3) (layers "F.Cu" "B.Cu") (free yes) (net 7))
 (via (at 124.054916 154.749) (size 0.6) (drill 0.3) (layers "F.Cu" "B.Cu") (free yes) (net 7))
 (via (at 128.554916 154.749) (size 0.6) (drill 0.3) (layers "F.Cu" "B.Cu") (free yes) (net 7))
 (via (at 127.054916 154.749) (size 0.6) (drill 0.3) (layers "F.Cu" "B.Cu") (free yes) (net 7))
 (segment (start 116.804916 155.404999) (end 116.779916 155.379999) (width 0.2) (layer "F.Cu") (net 47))
 (segment (start 116.904916 153.749001) (end 116.904916 153.404) (width 0.2) (layer "F.Cu") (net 47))
 (segment (start 116.804916 156.68) (end 116.804916 155.404999) (width 0.2) (layer "F.Cu") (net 47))
 (segment (start 116.779916 153.874001) (end 116.904916 153.749001) (width 0.2) (layer "F.Cu") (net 47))
 (segment (start 116.779916 155.379999) (end 116.779916 153.874001) (width 0.2) (layer "F.Cu") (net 47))
 (segment (start 116.304916 155.404999) (end 116.329916 155.379999) (width 0.2) (layer "F.Cu") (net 5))
 (segment (start 116.304916 156.68) (end 116.304916 155.404999) (width 0.2) (layer "F.Cu") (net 5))
 (segment (start 116.204916 153.749001) (end 116.204916 153.404) (width 0.2) (layer "F.Cu") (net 5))
 (segment (start 116.329916 153.874001) (end 116.204916 153.749001) (width 0.2) (layer "F.Cu") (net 5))
 (segment (start 116.329916 155.379999) (end 116.329916 153.874001) (width 0.2) (layer "F.Cu") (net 5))
 (segment (start 122.779916 155.379999) (end 122.779916 153.874001) (width 0.2) (layer "F.Cu") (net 1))
 (segment (start 122.779916 153.874001) (end 122.904916 153.749001) (width 0.2) (layer "F.Cu") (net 1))
 (segment (start 122.804916 155.404999) (end 122.779916 155.379999) (width 0.2) (layer "F.Cu") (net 1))
 (segment (start 122.904916 153.749001) (end 122.904916 153.404) (width 0.2) (layer "F.Cu") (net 1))
 (segment (start 122.804916 156.68) (end 122.804916 155.404999) (width 0.2) (layer "F.Cu") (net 1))
 (segment (start 122.329916 155.379999) (end 122.329916 153.874001) (width 0.2) (layer "F.Cu") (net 3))
 (segment (start 122.204916 153.749001) (end 122.204916 153.404) (width 0.2) (layer "F.Cu") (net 3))
 (segment (start 122.329916 153.874001) (end 122.204916 153.749001) (width 0.2) (layer "F.Cu") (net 3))
 (segment (start 122.304916 155.404999) (end 122.329916 155.379999) (width 0.2) (layer "F.Cu") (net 3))
 (segment (start 122.304916 156.68) (end 122.304916 155.404999) (width 0.2) (layer "F.Cu") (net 3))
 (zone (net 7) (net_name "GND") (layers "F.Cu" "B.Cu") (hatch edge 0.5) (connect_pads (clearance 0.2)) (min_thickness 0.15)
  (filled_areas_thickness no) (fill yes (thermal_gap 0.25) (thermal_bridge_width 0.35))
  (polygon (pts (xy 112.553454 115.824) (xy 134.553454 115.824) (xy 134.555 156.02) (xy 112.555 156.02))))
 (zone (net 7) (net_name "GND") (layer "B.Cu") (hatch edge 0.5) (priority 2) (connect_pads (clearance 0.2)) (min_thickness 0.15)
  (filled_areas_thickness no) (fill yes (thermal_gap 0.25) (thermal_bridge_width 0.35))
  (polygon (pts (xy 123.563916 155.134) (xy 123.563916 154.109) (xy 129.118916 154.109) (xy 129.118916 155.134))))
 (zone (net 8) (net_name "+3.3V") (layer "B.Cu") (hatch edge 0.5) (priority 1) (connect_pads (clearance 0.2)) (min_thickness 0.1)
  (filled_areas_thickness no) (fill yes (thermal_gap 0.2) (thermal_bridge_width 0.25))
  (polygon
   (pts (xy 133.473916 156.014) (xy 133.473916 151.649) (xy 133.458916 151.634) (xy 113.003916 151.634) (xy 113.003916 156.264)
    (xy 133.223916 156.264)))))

